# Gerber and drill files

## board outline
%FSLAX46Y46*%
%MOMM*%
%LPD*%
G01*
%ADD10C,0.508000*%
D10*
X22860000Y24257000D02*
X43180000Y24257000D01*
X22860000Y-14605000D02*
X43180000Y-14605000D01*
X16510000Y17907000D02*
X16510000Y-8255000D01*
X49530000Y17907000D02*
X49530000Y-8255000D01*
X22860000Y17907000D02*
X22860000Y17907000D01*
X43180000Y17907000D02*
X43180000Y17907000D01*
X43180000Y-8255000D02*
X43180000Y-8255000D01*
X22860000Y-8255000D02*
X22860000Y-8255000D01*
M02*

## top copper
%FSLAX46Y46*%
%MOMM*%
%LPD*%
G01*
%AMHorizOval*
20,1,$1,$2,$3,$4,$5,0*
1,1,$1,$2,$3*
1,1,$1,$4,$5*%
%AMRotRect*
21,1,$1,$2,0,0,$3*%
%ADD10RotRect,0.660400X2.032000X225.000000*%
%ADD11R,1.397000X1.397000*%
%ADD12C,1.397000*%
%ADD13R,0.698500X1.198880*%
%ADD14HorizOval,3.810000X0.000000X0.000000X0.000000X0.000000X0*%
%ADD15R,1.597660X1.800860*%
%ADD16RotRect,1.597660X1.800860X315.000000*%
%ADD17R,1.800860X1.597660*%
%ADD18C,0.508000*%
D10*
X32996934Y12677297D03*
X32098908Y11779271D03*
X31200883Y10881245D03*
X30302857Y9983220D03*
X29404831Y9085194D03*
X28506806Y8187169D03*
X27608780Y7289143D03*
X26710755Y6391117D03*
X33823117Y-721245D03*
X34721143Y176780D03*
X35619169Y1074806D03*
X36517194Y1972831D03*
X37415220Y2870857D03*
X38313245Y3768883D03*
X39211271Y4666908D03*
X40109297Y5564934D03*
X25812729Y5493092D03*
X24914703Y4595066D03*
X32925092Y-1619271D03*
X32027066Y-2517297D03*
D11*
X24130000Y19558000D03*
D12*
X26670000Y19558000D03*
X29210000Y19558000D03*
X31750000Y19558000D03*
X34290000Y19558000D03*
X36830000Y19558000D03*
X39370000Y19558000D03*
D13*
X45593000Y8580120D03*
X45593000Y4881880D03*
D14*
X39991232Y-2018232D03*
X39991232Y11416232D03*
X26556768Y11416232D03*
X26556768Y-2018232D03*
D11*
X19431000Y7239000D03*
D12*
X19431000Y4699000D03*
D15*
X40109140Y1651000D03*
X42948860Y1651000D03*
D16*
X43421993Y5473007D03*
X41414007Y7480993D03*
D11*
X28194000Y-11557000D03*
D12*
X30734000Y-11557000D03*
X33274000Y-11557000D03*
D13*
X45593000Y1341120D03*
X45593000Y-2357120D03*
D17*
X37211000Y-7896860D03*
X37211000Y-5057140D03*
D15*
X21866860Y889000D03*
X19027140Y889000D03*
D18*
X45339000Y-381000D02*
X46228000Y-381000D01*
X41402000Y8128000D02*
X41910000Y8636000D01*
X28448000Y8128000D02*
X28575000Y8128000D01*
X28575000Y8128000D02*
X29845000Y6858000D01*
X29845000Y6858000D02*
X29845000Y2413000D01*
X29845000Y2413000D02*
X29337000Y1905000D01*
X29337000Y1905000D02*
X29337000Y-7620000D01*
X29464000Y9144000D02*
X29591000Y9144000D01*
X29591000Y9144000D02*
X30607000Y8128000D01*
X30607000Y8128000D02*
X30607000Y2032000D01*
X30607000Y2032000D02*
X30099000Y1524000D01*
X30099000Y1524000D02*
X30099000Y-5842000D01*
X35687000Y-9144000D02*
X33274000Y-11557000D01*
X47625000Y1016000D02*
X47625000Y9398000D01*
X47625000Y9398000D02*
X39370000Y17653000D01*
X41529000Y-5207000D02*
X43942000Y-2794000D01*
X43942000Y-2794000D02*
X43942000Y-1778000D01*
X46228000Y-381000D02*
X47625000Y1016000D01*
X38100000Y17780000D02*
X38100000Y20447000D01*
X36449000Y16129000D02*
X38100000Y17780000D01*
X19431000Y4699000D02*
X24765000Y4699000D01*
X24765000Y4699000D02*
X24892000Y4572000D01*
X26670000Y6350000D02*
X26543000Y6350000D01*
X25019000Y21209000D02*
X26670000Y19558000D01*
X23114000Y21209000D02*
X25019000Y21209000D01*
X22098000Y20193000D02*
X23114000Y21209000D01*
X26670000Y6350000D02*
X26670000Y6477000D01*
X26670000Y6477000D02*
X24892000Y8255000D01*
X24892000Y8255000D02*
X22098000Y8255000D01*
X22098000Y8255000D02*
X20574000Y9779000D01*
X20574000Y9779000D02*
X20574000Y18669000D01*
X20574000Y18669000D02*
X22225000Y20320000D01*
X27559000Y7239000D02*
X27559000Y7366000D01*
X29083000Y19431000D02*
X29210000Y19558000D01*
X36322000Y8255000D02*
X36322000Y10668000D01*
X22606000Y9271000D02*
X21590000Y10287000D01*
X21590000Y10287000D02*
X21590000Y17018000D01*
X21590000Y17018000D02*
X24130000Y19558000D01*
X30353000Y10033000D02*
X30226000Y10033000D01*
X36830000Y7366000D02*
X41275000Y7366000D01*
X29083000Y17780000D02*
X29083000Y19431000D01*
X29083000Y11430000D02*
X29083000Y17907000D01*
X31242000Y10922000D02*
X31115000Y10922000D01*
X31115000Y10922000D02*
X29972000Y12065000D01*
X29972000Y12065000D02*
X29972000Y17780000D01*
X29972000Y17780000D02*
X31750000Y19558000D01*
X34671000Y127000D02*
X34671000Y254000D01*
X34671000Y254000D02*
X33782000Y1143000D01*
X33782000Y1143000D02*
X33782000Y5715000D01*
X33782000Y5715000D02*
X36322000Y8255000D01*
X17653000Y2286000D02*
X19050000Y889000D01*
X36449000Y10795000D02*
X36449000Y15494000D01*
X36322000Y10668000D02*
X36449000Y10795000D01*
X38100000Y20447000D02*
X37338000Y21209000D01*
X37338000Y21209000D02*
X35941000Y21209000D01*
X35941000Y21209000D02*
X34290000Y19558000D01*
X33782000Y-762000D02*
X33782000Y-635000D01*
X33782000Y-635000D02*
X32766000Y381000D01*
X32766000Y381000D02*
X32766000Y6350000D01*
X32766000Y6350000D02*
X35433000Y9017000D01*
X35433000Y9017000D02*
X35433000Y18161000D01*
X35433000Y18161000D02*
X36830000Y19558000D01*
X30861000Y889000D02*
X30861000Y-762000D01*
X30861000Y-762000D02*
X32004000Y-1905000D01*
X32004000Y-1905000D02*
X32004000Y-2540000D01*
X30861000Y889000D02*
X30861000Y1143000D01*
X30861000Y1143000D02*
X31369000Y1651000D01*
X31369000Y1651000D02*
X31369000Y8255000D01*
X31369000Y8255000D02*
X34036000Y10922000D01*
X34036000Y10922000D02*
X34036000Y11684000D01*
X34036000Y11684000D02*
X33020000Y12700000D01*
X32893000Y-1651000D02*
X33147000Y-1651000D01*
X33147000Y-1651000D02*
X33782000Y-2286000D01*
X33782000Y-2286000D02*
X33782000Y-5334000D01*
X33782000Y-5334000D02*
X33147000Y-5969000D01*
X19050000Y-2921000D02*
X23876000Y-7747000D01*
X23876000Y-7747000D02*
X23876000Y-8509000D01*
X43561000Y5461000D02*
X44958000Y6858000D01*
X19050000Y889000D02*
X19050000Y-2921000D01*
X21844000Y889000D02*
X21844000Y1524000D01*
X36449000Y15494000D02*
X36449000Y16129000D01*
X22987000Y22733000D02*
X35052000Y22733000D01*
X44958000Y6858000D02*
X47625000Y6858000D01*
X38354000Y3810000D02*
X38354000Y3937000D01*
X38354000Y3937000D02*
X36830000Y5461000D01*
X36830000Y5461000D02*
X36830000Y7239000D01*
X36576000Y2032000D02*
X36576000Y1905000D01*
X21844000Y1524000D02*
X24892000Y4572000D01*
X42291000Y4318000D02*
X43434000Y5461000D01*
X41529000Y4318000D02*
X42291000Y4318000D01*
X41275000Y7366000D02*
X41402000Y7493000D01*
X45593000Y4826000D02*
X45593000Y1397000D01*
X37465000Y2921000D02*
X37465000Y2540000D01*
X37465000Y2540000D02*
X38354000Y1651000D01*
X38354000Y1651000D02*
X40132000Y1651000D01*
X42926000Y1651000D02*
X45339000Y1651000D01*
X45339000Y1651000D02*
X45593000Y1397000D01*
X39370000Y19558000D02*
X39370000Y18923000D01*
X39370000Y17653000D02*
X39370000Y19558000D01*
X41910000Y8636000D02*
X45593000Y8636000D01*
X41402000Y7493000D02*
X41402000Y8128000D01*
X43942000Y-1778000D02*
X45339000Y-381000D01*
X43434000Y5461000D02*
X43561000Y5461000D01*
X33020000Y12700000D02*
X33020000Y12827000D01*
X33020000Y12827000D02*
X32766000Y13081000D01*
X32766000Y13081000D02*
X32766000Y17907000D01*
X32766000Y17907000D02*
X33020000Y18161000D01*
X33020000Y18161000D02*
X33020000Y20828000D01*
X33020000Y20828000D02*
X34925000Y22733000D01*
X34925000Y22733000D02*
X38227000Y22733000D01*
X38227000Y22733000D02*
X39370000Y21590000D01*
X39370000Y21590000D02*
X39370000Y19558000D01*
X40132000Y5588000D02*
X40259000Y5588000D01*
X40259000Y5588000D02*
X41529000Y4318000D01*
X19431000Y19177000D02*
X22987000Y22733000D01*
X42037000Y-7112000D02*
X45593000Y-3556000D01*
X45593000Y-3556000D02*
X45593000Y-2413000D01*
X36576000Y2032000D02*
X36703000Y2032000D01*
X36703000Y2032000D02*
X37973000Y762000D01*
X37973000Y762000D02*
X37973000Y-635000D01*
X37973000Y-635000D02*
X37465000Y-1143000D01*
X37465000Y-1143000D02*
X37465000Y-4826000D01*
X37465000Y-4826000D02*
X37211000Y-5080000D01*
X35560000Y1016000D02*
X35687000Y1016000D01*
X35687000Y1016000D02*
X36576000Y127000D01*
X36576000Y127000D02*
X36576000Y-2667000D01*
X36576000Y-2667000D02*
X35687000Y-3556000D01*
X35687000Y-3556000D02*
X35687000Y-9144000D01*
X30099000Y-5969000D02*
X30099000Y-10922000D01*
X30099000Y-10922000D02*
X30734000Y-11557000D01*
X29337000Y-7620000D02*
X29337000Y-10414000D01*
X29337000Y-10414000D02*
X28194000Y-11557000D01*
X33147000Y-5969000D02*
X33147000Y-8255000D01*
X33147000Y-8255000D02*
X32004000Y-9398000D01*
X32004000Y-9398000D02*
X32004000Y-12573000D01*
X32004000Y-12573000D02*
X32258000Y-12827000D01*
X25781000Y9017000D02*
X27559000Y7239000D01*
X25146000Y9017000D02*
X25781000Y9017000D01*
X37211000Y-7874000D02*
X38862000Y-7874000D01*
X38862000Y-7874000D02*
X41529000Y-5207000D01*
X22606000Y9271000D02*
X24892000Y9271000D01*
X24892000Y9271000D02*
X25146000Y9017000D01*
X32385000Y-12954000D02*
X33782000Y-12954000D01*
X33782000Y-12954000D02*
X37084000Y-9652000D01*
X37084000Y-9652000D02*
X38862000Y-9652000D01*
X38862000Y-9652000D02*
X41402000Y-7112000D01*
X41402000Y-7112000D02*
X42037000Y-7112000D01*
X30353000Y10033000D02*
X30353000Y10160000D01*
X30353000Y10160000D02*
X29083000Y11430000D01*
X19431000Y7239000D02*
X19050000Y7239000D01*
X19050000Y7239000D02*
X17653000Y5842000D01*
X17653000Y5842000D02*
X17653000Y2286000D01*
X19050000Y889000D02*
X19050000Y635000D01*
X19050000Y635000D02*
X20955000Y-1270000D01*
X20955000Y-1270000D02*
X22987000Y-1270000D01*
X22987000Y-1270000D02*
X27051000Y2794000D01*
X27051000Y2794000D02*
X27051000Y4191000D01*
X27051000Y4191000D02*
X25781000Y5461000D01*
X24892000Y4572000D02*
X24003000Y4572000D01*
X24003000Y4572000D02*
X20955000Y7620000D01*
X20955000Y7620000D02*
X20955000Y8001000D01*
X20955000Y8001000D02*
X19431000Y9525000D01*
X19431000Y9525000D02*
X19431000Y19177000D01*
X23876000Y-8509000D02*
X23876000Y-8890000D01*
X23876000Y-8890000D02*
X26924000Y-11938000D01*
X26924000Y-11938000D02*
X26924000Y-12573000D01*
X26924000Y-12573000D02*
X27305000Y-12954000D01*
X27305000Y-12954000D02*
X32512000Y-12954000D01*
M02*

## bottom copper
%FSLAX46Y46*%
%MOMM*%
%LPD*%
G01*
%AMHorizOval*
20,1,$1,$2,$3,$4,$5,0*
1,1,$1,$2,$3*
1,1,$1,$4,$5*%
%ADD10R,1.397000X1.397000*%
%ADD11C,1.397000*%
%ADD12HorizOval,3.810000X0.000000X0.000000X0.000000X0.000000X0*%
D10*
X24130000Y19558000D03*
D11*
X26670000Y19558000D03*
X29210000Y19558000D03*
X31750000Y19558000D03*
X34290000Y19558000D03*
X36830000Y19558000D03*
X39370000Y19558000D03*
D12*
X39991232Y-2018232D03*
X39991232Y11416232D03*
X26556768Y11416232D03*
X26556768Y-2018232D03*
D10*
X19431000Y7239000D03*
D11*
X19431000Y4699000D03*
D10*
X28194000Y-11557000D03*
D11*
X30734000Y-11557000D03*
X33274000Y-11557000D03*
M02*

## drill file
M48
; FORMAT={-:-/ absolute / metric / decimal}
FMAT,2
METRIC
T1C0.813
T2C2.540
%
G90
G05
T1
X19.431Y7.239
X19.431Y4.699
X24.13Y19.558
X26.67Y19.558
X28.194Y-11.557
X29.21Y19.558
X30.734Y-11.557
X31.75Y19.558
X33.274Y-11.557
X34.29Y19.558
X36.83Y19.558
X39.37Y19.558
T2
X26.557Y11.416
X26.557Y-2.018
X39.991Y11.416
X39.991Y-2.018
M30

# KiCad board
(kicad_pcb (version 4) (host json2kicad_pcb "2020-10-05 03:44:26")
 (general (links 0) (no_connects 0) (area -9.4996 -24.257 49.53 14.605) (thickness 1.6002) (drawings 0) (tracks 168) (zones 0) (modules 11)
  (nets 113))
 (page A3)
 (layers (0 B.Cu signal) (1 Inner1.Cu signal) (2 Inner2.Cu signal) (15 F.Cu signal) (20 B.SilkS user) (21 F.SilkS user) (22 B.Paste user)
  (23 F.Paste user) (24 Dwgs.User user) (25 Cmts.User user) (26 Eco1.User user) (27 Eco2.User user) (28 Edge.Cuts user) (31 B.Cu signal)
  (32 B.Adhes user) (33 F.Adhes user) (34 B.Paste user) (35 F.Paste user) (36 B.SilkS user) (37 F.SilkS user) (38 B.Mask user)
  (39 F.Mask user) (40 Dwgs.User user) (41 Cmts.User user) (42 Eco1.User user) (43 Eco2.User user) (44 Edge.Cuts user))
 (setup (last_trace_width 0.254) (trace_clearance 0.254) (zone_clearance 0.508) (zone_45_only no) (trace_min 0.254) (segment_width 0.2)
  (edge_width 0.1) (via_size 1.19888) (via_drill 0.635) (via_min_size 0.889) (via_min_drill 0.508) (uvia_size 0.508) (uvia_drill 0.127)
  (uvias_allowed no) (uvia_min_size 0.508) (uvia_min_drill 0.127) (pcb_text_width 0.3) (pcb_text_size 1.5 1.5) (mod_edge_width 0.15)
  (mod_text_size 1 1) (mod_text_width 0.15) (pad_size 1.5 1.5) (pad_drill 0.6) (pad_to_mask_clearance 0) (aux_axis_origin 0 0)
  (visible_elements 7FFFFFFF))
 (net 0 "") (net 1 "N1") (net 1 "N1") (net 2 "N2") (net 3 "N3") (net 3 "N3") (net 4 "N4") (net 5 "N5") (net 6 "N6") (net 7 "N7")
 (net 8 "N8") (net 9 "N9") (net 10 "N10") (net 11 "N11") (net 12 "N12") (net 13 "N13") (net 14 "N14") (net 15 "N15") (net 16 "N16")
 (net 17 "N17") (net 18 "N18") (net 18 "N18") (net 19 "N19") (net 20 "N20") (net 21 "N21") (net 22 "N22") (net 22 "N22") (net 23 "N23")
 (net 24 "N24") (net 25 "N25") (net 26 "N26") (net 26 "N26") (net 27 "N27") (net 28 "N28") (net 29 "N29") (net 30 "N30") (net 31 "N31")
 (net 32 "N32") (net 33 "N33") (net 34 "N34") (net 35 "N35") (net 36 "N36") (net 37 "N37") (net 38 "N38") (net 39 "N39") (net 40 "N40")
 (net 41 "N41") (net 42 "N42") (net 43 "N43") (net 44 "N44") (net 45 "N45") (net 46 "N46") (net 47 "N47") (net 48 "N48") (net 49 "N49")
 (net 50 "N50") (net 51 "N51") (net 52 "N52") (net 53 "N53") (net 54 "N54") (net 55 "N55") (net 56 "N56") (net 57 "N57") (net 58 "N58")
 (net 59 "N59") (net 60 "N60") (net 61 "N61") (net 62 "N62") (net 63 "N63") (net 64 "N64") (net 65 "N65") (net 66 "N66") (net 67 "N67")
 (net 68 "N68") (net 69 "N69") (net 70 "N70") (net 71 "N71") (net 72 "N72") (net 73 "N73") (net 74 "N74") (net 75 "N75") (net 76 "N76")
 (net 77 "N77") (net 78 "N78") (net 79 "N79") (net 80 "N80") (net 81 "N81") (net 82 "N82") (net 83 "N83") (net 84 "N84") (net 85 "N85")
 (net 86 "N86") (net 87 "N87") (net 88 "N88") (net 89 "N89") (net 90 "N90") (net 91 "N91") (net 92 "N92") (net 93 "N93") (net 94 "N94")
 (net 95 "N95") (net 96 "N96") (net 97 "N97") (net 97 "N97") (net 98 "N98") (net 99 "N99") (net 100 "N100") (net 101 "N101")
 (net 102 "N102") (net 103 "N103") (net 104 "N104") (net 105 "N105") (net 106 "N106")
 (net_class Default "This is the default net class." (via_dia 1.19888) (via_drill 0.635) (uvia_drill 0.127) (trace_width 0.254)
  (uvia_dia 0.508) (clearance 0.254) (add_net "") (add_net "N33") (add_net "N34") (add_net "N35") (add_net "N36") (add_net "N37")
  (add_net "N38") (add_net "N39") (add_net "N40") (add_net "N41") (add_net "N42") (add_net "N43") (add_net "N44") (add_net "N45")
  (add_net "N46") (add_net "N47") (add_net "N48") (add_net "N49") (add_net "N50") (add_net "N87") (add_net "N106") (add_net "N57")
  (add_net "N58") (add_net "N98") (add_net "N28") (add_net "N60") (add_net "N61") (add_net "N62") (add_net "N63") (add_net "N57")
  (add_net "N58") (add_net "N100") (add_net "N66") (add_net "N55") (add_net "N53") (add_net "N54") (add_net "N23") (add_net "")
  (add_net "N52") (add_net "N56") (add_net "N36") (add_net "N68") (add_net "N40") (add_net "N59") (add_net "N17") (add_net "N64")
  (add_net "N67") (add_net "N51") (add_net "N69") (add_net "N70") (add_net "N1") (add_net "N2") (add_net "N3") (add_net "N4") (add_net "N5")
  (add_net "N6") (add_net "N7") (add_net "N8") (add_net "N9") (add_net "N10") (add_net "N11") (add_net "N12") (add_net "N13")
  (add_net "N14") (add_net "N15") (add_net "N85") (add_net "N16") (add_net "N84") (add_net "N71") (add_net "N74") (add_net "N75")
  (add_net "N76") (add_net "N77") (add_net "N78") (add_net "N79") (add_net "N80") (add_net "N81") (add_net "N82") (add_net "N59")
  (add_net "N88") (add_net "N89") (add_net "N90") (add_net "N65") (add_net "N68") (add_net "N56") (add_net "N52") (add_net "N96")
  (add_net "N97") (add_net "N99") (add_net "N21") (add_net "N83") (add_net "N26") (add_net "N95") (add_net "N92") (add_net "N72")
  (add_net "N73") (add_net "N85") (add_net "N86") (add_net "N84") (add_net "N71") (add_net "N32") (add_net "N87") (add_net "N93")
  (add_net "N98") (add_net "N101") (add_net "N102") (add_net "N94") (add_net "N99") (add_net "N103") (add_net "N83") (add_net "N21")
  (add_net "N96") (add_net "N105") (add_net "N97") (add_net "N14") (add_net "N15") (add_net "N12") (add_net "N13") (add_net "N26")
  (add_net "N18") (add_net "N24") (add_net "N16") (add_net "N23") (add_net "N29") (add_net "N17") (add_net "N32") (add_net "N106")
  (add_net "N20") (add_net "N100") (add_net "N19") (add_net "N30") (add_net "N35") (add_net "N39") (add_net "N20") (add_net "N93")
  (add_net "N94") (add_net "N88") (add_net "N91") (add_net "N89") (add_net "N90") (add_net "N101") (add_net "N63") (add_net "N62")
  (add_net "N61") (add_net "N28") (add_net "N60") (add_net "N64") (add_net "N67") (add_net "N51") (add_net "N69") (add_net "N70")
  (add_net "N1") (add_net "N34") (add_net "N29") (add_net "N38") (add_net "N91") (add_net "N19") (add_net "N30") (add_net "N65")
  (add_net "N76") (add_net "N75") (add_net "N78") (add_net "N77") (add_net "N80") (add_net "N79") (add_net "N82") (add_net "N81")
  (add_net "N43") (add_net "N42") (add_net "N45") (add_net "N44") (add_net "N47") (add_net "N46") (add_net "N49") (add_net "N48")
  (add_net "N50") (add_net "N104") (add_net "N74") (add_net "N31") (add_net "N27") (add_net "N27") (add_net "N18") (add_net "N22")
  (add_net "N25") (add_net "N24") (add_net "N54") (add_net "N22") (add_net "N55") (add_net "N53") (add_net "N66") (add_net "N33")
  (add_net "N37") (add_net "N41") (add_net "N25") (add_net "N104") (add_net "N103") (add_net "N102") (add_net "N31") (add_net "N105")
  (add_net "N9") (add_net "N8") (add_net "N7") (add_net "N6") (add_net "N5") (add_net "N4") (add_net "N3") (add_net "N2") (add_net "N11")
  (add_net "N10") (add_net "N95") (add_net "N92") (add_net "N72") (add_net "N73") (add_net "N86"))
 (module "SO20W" (layer "F.Cu") (at 32.512 -5.08 -135.00)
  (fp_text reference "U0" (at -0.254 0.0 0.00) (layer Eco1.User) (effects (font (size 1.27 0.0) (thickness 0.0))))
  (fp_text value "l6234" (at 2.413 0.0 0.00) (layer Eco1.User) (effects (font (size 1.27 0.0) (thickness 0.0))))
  (pad 1 smd rect (at -5.715 5.0292 -135.00) (size 0.6604 2.032) (drill 0.0) (layers "F.Cu" "F.Paste") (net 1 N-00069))
  (pad 2 smd rect (at -4.445 5.0292 -135.00) (size 0.6604 2.032) (drill 0.0) (layers "F.Cu" "F.Paste") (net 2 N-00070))
  (pad 3 smd rect (at -3.175 5.0292 -135.00) (size 0.6604 2.032) (drill 0.0) (layers "F.Cu" "F.Paste") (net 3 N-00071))
  (pad 4 smd rect (at -1.905 5.0292 -135.00) (size 0.6604 2.032) (drill 0.0) (layers "F.Cu" "F.Paste") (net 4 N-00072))
  (pad 5 smd rect (at -0.635 5.0292 -135.00) (size 0.6604 2.032) (drill 0.0) (layers "F.Cu" "F.Paste") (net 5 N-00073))
  (pad 6 smd rect (at 0.635 5.0292 -135.00) (size 0.6604 2.032) (drill 0.0) (layers "F.Cu" "F.Paste") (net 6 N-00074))
  (pad 7 smd rect (at 1.905 5.0292 -135.00) (size 0.6604 2.032) (drill 0.0) (layers "F.Cu" "F.Paste") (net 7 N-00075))
  (pad 8 smd rect (at 3.175 5.0292 -135.00) (size 0.6604 2.032) (drill 0.0) (layers "F.Cu" "F.Paste") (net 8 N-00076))
  (pad 13 smd rect (at 3.175 -5.0292 -135.00) (size 0.6604 2.032) (drill 0.0) (layers "F.Cu" "F.Paste") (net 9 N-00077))
  (pad 14 smd rect (at 1.905 -5.0292 -135.00) (size 0.6604 2.032) (drill 0.0) (layers "F.Cu" "F.Paste") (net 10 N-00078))
  (pad 15 smd rect (at 0.635 -5.0292 -135.00) (size 0.6604 2.032) (drill 0.0) (layers "F.Cu" "F.Paste") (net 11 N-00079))
  (pad 16 smd rect (at -0.635 -5.0292 -135.00) (size 0.6604 2.032) (drill 0.0) (layers "F.Cu" "F.Paste") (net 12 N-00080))
  (pad 17 smd rect (at -1.905 -5.0292 -135.00) (size 0.6604 2.032) (drill 0.0) (layers "F.Cu" "F.Paste") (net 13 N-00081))
  (pad 18 smd rect (at -3.175 -5.0292 -135.00) (size 0.6604 2.032) (drill 0.0) (layers "F.Cu" "F.Paste") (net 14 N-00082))
  (pad 19 smd rect (at -4.445 -5.0292 -135.00) (size 0.6604 2.032) (drill 0.0) (layers "F.Cu" "F.Paste") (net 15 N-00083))
  (pad 20 smd rect (at -5.715 -5.0292 -135.00) (size 0.6604 2.032) (drill 0.0) (layers "F.Cu" "F.Paste") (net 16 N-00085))
  (pad 9 smd rect (at 4.445 5.0292 -135.00) (size 0.6604 2.032) (drill 0.0) (layers "F.Cu" "F.Paste") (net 16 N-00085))
  (pad 10 smd rect (at 5.715 5.0292 -135.00) (size 0.6604 2.032) (drill 0.0) (layers "F.Cu" "F.Paste") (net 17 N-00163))
  (pad 12 smd rect (at 4.445 -5.0292 -135.00) (size 0.6604 2.032) (drill 0.0) (layers "F.Cu" "F.Paste") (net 6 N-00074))
  (pad 11 smd rect (at 5.715 -5.0292 -135.00) (size 0.6604 2.032) (drill 0.0) (layers "F.Cu" "F.Paste") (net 1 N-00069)))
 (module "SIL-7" (layer "F.Cu") (at 31.75 -19.558 0.00)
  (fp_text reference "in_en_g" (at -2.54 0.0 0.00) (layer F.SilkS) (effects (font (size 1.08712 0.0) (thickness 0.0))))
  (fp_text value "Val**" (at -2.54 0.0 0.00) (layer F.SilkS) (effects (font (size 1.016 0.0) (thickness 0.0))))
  (pad 1 thru_hole rect (at -7.62 0.0 0.00) (size 1.397 1.397) (drill 0.8128)
   (layers "B.Cu" "Inner1.Cu" "Inner2.Cu" "F.Cu" "F.SilkS" "B.Paste" "F.Paste") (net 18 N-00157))
  (pad 2 thru_hole circle (at -5.08 0.0 0.00) (size 1.397 1.397) (drill 0.8128)
   (layers "B.Cu" "Inner1.Cu" "Inner2.Cu" "F.Cu" "B.SilkS" "F.SilkS" "B.Paste" "F.Paste") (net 8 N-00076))
  (pad 3 thru_hole circle (at -2.54 0.0 0.00) (size 1.397 1.397) (drill 0.8128)
   (layers "B.Cu" "Inner1.Cu" "Inner2.Cu" "F.Cu" "B.SilkS" "F.SilkS" "B.Paste" "F.Paste") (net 7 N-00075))
  (pad 4 thru_hole circle (at 0.0 0.0 0.00) (size 1.397 1.397) (drill 0.8128)
   (layers "B.Cu" "Inner1.Cu" "Inner2.Cu" "F.Cu" "B.SilkS" "F.SilkS" "B.Paste" "F.Paste") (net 3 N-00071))
  (pad 5 thru_hole circle (at 2.54 0.0 0.00) (size 1.397 1.397) (drill 0.8128)
   (layers "B.Cu" "Inner1.Cu" "Inner2.Cu" "F.Cu" "B.SilkS" "F.SilkS" "B.Paste" "F.Paste") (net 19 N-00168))
  (pad 6 thru_hole circle (at 5.08 0.0 0.00) (size 1.397 1.397) (drill 0.8128)
   (layers "B.Cu" "Inner1.Cu" "Inner2.Cu" "F.Cu" "B.SilkS" "F.SilkS" "B.Paste" "F.Paste") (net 9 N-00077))
  (pad 7 thru_hole circle (at 7.62 0.0 0.00) (size 1.397 1.397) (drill 0.8128)
   (layers "B.Cu" "Inner1.Cu" "Inner2.Cu" "F.Cu" "B.SilkS" "F.SilkS" "B.Paste" "F.Paste") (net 1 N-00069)))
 (segment (start 45.339 0.381) (end 46.228 0.381) (width 0.508) (layer F.Cu) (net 1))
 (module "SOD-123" (layer "F.Cu") (at 45.593 -6.731 -90.00)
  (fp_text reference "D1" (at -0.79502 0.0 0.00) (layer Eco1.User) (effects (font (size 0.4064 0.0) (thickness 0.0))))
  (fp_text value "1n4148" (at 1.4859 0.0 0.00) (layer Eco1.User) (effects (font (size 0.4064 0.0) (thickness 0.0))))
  (pad C smd rect (at -1.84912 0.0 -90.00) (size 1.19888 0.6985) (drill 0.0) (layers "F.Cu" "F.Paste") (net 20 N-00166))
  (pad A smd rect (at 1.84912 0.0 -90.00) (size 1.19888 0.6985) (drill 0.0) (layers "F.Cu" "F.Paste") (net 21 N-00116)))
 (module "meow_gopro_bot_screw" (layer "F.Cu") (at 33.274 -4.699 45.00)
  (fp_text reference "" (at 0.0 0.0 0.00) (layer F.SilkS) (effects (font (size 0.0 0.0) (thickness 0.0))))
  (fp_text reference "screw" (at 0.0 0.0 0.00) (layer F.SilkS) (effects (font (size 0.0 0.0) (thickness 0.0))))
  (pad S0 thru_hole oval (at 0.0 9.4996 45.00) (size 3.81 3.81) (drill 2.54)
   (layers "B.Cu" "Inner1.Cu" "Inner2.Cu" "F.Cu" "B.Paste" "F.Paste") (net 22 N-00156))
  (pad S1 thru_hole oval (at 9.4996 0.0 45.00) (size 3.81 3.81) (drill 2.54)
   (layers "B.Cu" "Inner1.Cu" "Inner2.Cu" "F.Cu" "B.Paste" "F.Paste") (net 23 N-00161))
  (pad S2 thru_hole oval (at 0.0 -9.4996 45.00) (size 3.81 3.81) (drill 2.54)
   (layers "B.Cu" "Inner1.Cu" "Inner2.Cu" "F.Cu" "B.Paste" "F.Paste") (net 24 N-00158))
  (pad S3 thru_hole oval (at -9.4996 0.0 45.00) (size 3.81 3.81) (drill 2.54)
   (layers "B.Cu" "Inner1.Cu" "Inner2.Cu" "F.Cu" "B.Paste" "F.Paste") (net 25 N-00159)))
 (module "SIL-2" (layer "F.Cu") (at 19.431 -5.969 -90.00)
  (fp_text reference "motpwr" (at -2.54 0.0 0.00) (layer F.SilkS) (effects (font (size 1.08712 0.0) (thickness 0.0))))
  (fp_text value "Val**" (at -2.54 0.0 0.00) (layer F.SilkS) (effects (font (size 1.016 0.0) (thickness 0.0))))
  (pad 1 thru_hole rect (at -1.27 0.0 -90.00) (size 1.397 1.397) (drill 0.8128)
   (layers "B.Cu" "Inner1.Cu" "Inner2.Cu" "F.Cu" "F.SilkS" "B.Paste" "F.Paste") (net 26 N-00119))
  (pad 2 thru_hole circle (at 1.27 0.0 -90.00) (size 1.397 1.397) (drill 0.8128)
   (layers "B.Cu" "Inner1.Cu" "Inner2.Cu" "F.Cu" "F.SilkS" "B.Paste" "F.Paste") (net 17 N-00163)))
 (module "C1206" (layer "F.Cu") (at 41.529 -1.651 180.00)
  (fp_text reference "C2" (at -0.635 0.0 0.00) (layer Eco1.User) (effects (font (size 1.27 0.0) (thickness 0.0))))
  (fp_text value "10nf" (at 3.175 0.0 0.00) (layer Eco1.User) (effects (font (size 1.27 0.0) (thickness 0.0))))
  (pad 2 smd rect (at 1.41986 0.0 -180.00) (size 1.59766 1.80086) (drill 0.0) (layers "F.Cu" "F.Paste") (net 13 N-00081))
  (pad 1 smd rect (at -1.41986 0.0 -180.00) (size 1.59766 1.80086) (drill 0.0) (layers "F.Cu" "F.Paste") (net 21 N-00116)))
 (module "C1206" (layer "F.Cu") (at 42.418 -6.477 -45.00)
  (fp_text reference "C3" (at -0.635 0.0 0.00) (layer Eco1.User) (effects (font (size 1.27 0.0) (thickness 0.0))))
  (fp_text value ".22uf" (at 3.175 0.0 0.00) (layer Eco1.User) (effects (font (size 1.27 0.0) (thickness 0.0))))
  (pad 2 smd rect (at 1.41986 0.0 -45.00) (size 1.59766 1.80086) (drill 0.0) (layers "F.Cu" "F.Paste") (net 16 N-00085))
  (pad 1 smd rect (at -1.41986 0.0 -45.00) (size 1.59766 1.80086) (drill 0.0) (layers "F.Cu" "F.Paste") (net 12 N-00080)))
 (segment (start 41.402 -8.128) (end 41.91 -8.636) (width 0.508) (layer F.Cu) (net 14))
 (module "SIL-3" (layer "F.Cu") (at 30.734 11.557 0.00)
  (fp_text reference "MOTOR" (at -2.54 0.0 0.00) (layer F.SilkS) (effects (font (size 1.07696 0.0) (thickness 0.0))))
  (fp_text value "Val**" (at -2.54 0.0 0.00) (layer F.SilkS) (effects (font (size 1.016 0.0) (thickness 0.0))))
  (pad 1 thru_hole rect (at -2.54 0.0 0.00) (size 1.397 1.397) (drill 0.8128)
   (layers "B.Cu" "Inner1.Cu" "Inner2.Cu" "F.Cu" "F.SilkS" "B.Paste" "F.Paste") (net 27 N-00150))
  (pad 2 thru_hole circle (at 0.0 0.0 0.00) (size 1.397 1.397) (drill 0.8128)
   (layers "B.Cu" "Inner1.Cu" "Inner2.Cu" "F.Cu" "F.SilkS" "B.Paste" "F.Paste") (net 5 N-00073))
  (pad 3 thru_hole circle (at 2.54 0.0 0.00) (size 1.397 1.397) (drill 0.8128)
   (layers "B.Cu" "Inner1.Cu" "Inner2.Cu" "F.Cu" "F.SilkS" "B.Paste" "F.Paste") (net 11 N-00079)))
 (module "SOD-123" (layer "F.Cu") (at 45.593 0.508 -90.00)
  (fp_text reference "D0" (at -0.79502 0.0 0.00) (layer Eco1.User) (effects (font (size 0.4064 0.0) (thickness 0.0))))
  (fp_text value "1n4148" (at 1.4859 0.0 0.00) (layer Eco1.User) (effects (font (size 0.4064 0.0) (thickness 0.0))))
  (pad C smd rect (at -1.84912 0.0 -90.00) (size 1.19888 0.6985) (drill 0.0) (layers "F.Cu" "F.Paste") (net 1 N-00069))
  (pad A smd rect (at 1.84912 0.0 -90.00) (size 1.19888 0.6985) (drill 0.0) (layers "F.Cu" "F.Paste") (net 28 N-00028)))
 (segment (start 28.448 -8.128) (end 28.575 -8.128) (width 0.508) (layer F.Cu) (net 6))
 (segment (start 28.575 -8.128) (end 29.845 -6.858) (width 0.508) (layer F.Cu) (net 6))
 (segment (start 29.845 -6.858) (end 29.845 -2.413) (width 0.508) (layer F.Cu) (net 6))
 (segment (start 29.845 -2.413) (end 29.337 -1.905) (width 0.508) (layer F.Cu) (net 6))
 (segment (start 29.337 -1.905) (end 29.337 7.62) (width 0.508) (layer F.Cu) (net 6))
 (segment (start 29.464 -9.144) (end 29.591 -9.144) (width 0.508) (layer F.Cu) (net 5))
 (segment (start 29.591 -9.144) (end 30.607 -8.128) (width 0.508) (layer F.Cu) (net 5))
 (segment (start 30.607 -8.128) (end 30.607 -2.032) (width 0.508) (layer F.Cu) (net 5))
 (segment (start 30.607 -2.032) (end 30.099 -1.524) (width 0.508) (layer F.Cu) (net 5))
 (segment (start 30.099 -1.524) (end 30.099 5.842) (width 0.508) (layer F.Cu) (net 5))
 (segment (start 35.687 9.144) (end 33.274 11.557) (width 0.508) (layer F.Cu) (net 11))
 (segment (start 47.625 -1.016) (end 47.625 -9.398) (width 0.508) (layer F.Cu) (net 1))
 (segment (start 47.625 -9.398) (end 39.37 -17.653) (width 0.508) (layer F.Cu) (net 1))
 (segment (start 41.529 5.207) (end 43.942 2.794) (width 0.508) (layer F.Cu) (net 1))
 (segment (start 43.942 2.794) (end 43.942 1.778) (width 0.508) (layer F.Cu) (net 1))
 (segment (start 46.228 0.381) (end 47.625 -1.016) (width 0.508) (layer F.Cu) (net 1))
 (segment (start 38.1 -17.78) (end 38.1 -20.447) (width 0.508) (layer F.Cu) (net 10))
 (segment (start 36.449 -16.129) (end 38.1 -17.78) (width 0.508) (layer F.Cu) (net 10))
 (segment (start 19.431 -4.699) (end 24.765 -4.699) (width 0.508) (layer F.Cu) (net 17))
 (segment (start 24.765 -4.699) (end 24.892 -4.572) (width 0.508) (layer F.Cu) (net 17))
 (segment (start 26.67 -6.35) (end 26.543 -6.35) (width 0.508) (layer F.Cu) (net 8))
 (segment (start 25.019 -21.209) (end 26.67 -19.558) (width 0.508) (layer F.Cu) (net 8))
 (segment (start 23.114 -21.209) (end 25.019 -21.209) (width 0.508) (layer F.Cu) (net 8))
 (segment (start 22.098 -20.193) (end 23.114 -21.209) (width 0.508) (layer F.Cu) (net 8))
 (segment (start 26.67 -6.35) (end 26.67 -6.477) (width 0.508) (layer F.Cu) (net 8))
 (segment (start 26.67 -6.477) (end 24.892 -8.255) (width 0.508) (layer F.Cu) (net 8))
 (segment (start 24.892 -8.255) (end 22.098 -8.255) (width 0.508) (layer F.Cu) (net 8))
 (segment (start 22.098 -8.255) (end 20.574 -9.779) (width 0.508) (layer F.Cu) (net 8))
 (segment (start 20.574 -9.779) (end 20.574 -18.669) (width 0.508) (layer F.Cu) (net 8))
 (segment (start 20.574 -18.669) (end 22.225 -20.32) (width 0.508) (layer F.Cu) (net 8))
 (segment (start 27.559 -7.239) (end 27.559 -7.366) (width 0.508) (layer F.Cu) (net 7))
 (segment (start 29.083 -19.431) (end 29.21 -19.558) (width 0.508) (layer F.Cu) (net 4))
 (segment (start 36.322 -8.255) (end 36.322 -10.668) (width 0.508) (layer F.Cu) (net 10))
 (segment (start 22.606 -9.271) (end 21.59 -10.287) (width 0.508) (layer F.Cu) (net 18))
 (segment (start 21.59 -10.287) (end 21.59 -17.018) (width 0.508) (layer F.Cu) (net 18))
 (segment (start 21.59 -17.018) (end 24.13 -19.558) (width 0.508) (layer F.Cu) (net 18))
 (segment (start 30.353 -10.033) (end 30.226 -10.033) (width 0.508) (layer F.Cu) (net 4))
 (segment (start 36.83 -7.366) (end 41.275 -7.366) (width 0.508) (layer F.Cu) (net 14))
 (segment (start 29.083 -17.78) (end 29.083 -19.431) (width 0.508) (layer F.Cu) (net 4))
 (segment (start 29.083 -11.43) (end 29.083 -17.907) (width 0.508) (layer F.Cu) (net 4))
 (segment (start 31.242 -10.922) (end 31.115 -10.922) (width 0.508) (layer F.Cu) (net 3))
 (segment (start 31.115 -10.922) (end 29.972 -12.065) (width 0.508) (layer F.Cu) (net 3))
 (segment (start 29.972 -12.065) (end 29.972 -17.78) (width 0.508) (layer F.Cu) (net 3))
 (segment (start 29.972 -17.78) (end 31.75 -19.558) (width 0.508) (layer F.Cu) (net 3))
 (segment (start 34.671 -0.127) (end 34.671 -0.254) (width 0.508) (layer F.Cu) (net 10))
 (segment (start 34.671 -0.254) (end 33.782 -1.143) (width 0.508) (layer F.Cu) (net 10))
 (segment (start 33.782 -1.143) (end 33.782 -5.715) (width 0.508) (layer F.Cu) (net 10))
 (segment (start 33.782 -5.715) (end 36.322 -8.255) (width 0.508) (layer F.Cu) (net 10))
 (segment (start 17.653 -2.286) (end 19.05 -0.889) (width 0.508) (layer F.Cu) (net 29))
 (segment (start 36.449 -10.795) (end 36.449 -15.494) (width 0.508) (layer F.Cu) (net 10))
 (segment (start 36.322 -10.668) (end 36.449 -10.795) (width 0.508) (layer F.Cu) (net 10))
 (segment (start 38.1 -20.447) (end 37.338 -21.209) (width 0.508) (layer F.Cu) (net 19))
 (segment (start 37.338 -21.209) (end 35.941 -21.209) (width 0.508) (layer F.Cu) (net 19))
 (segment (start 35.941 -21.209) (end 34.29 -19.558) (width 0.508) (layer F.Cu) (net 19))
 (segment (start 33.782 0.762) (end 33.782 0.635) (width 0.508) (layer F.Cu) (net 9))
 (segment (start 33.782 0.635) (end 32.766 -0.381) (width 0.508) (layer F.Cu) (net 9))
 (segment (start 32.766 -0.381) (end 32.766 -6.35) (width 0.508) (layer F.Cu) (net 9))
 (segment (start 32.766 -6.35) (end 35.433 -9.017) (width 0.508) (layer F.Cu) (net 9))
 (segment (start 35.433 -9.017) (end 35.433 -18.161) (width 0.508) (layer F.Cu) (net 9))
 (segment (start 35.433 -18.161) (end 36.83 -19.558) (width 0.508) (layer F.Cu) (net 9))
 (segment (start 30.861 -0.889) (end 30.861 0.762) (width 0.508) (layer F.Cu) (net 1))
 (segment (start 30.861 0.762) (end 32.004 1.905) (width 0.508) (layer F.Cu) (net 1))
 (segment (start 32.004 1.905) (end 32.004 2.54) (width 0.508) (layer F.Cu) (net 1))
 (segment (start 30.861 -0.889) (end 30.861 -1.143) (width 0.508) (layer F.Cu) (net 1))
 (segment (start 30.861 -1.143) (end 31.369 -1.651) (width 0.508) (layer F.Cu) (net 1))
 (segment (start 31.369 -1.651) (end 31.369 -8.255) (width 0.508) (layer F.Cu) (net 1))
 (segment (start 31.369 -8.255) (end 34.036 -10.922) (width 0.508) (layer F.Cu) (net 1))
 (segment (start 34.036 -10.922) (end 34.036 -11.684) (width 0.508) (layer F.Cu) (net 1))
 (segment (start 34.036 -11.684) (end 33.02 -12.7) (width 0.508) (layer F.Cu) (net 1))
 (segment (start 32.893 1.651) (end 33.147 1.651) (width 0.508) (layer F.Cu) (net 6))
 (segment (start 33.147 1.651) (end 33.782 2.286) (width 0.508) (layer F.Cu) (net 6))
 (segment (start 33.782 2.286) (end 33.782 5.334) (width 0.508) (layer F.Cu) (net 6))
 (segment (start 33.782 5.334) (end 33.147 5.969) (width 0.508) (layer F.Cu) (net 6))
 (segment (start 19.05 2.921) (end 23.876 7.747) (width 0.508) (layer F.Cu) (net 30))
 (segment (start 23.876 7.747) (end 23.876 8.509) (width 0.508) (layer F.Cu) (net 30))
 (segment (start 43.561 -5.461) (end 44.958 -6.858) (width 0.508) (layer F.Cu) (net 1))
 (segment (start 19.05 -0.889) (end 19.05 2.921) (width 0.508) (layer F.Cu) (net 30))
 (segment (start 21.844 -0.889) (end 21.844 -1.524) (width 0.508) (layer F.Cu) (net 17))
 (segment (start 36.449 -15.494) (end 36.449 -16.129) (width 0.508) (layer F.Cu) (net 10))
 (segment (start 22.987 -22.733) (end 35.052 -22.733) (width 0.508) (layer F.Cu) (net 1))
 (segment (start 44.958 -6.858) (end 47.625 -6.858) (width 0.508) (layer F.Cu) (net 1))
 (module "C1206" (layer "F.Cu") (at 37.211 6.477 -90.00)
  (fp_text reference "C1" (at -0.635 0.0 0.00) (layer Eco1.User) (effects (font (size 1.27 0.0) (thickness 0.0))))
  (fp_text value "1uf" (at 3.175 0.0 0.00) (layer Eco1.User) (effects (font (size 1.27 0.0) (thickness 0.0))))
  (pad 2 smd rect (at 1.41986 0.0 -90.00) (size 1.59766 1.80086) (drill 0.0) (layers "F.Cu" "F.Paste") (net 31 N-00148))
  (pad 1 smd rect (at -1.41986 0.0 -90.00) (size 1.59766 1.80086) (drill 0.0) (layers "F.Cu" "F.Paste") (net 29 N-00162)))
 (segment (start 38.354 -3.81) (end 38.354 -3.937) (width 0.508) (layer F.Cu) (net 14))
 (segment (start 38.354 -3.937) (end 36.83 -5.461) (width 0.508) (layer F.Cu) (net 14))
 (segment (start 36.83 -5.461) (end 36.83 -7.239) (width 0.508) (layer F.Cu) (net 14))
 (segment (start 36.576 -2.032) (end 36.576 -1.905) (width 0.508) (layer F.Cu) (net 12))
 (segment (start 21.844 -1.524) (end 24.892 -4.572) (width 0.508) (layer F.Cu) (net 17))
 (segment (start 42.291 -4.318) (end 43.434 -5.461) (width 0.508) (layer F.Cu) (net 16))
 (segment (start 41.529 -4.318) (end 42.291 -4.318) (width 0.508) (layer F.Cu) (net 16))
 (segment (start 41.275 -7.366) (end 41.402 -7.493) (width 0.508) (layer F.Cu) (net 14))
 (segment (start 45.593 -4.826) (end 45.593 -1.397) (width 0.508) (layer F.Cu) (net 21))
 (segment (start 37.465 -2.921) (end 37.465 -2.54) (width 0.508) (layer F.Cu) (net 13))
 (segment (start 37.465 -2.54) (end 38.354 -1.651) (width 0.508) (layer F.Cu) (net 13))
 (segment (start 38.354 -1.651) (end 40.132 -1.651) (width 0.508) (layer F.Cu) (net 13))
 (segment (start 42.926 -1.651) (end 45.339 -1.651) (width 0.508) (layer F.Cu) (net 21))
 (segment (start 45.339 -1.651) (end 45.593 -1.397) (width 0.508) (layer F.Cu) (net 21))
 (segment (start 39.37 -19.558) (end 39.37 -18.923) (width 0.508) (layer F.Cu) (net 1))
 (segment (start 39.37 -17.653) (end 39.37 -19.558) (width 0.508) (layer F.Cu) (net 1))
 (segment (start 41.91 -8.636) (end 45.593 -8.636) (width 0.508) (layer F.Cu) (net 14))
 (segment (start 41.402 -7.493) (end 41.402 -8.128) (width 0.508) (layer F.Cu) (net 14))
 (segment (start 43.942 1.778) (end 45.339 0.381) (width 0.508) (layer F.Cu) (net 1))
 (segment (start 43.434 -5.461) (end 43.561 -5.461) (width 0.508) (layer F.Cu) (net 1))
 (segment (start 33.02 -12.7) (end 33.02 -12.827) (width 0.508) (layer F.Cu) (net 1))
 (segment (start 33.02 -12.827) (end 32.766 -13.081) (width 0.508) (layer F.Cu) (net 1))
 (segment (start 32.766 -13.081) (end 32.766 -17.907) (width 0.508) (layer F.Cu) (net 1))
 (segment (start 32.766 -17.907) (end 33.02 -18.161) (width 0.508) (layer F.Cu) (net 1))
 (segment (start 33.02 -18.161) (end 33.02 -20.828) (width 0.508) (layer F.Cu) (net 1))
 (segment (start 33.02 -20.828) (end 34.925 -22.733) (width 0.508) (layer F.Cu) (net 1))
 (segment (start 34.925 -22.733) (end 38.227 -22.733) (width 0.508) (layer F.Cu) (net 1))
 (segment (start 38.227 -22.733) (end 39.37 -21.59) (width 0.508) (layer F.Cu) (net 1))
 (segment (start 39.37 -21.59) (end 39.37 -19.558) (width 0.508) (layer F.Cu) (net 1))
 (segment (start 40.132 -5.588) (end 40.259 -5.588) (width 0.508) (layer F.Cu) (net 16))
 (segment (start 40.259 -5.588) (end 41.529 -4.318) (width 0.508) (layer F.Cu) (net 16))
 (segment (start 19.431 -19.177) (end 22.987 -22.733) (width 0.508) (layer F.Cu) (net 1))
 (segment (start 42.037 7.112) (end 45.593 3.556) (width 0.508) (layer F.Cu) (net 1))
 (segment (start 45.593 3.556) (end 45.593 2.413) (width 0.508) (layer F.Cu) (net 1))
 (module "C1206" (layer "F.Cu") (at 20.447 -0.889 0.00)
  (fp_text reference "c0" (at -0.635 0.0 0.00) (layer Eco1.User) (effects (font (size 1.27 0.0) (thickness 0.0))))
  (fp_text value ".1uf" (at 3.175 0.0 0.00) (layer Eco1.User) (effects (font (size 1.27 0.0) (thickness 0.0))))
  (pad 2 smd rect (at 1.41986 0.0 0.00) (size 1.59766 1.80086) (drill 0.0) (layers "F.Cu" "F.Paste") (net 17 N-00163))
  (pad 1 smd rect (at -1.41986 0.0 0.00) (size 1.59766 1.80086) (drill 0.0) (layers "F.Cu" "F.Paste") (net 30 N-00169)))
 (segment (start 36.576 -2.032) (end 36.703 -2.032) (width 0.508) (layer F.Cu) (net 12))
 (segment (start 36.703 -2.032) (end 37.973 -0.762) (width 0.508) (layer F.Cu) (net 12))
 (segment (start 37.973 -0.762) (end 37.973 0.635) (width 0.508) (layer F.Cu) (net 12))
 (segment (start 37.973 0.635) (end 37.465 1.143) (width 0.508) (layer F.Cu) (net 12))
 (segment (start 37.465 1.143) (end 37.465 4.826) (width 0.508) (layer F.Cu) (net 12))
 (segment (start 37.465 4.826) (end 37.211 5.08) (width 0.508) (layer F.Cu) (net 12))
 (segment (start 35.56 -1.016) (end 35.687 -1.016) (width 0.508) (layer F.Cu) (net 11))
 (segment (start 35.687 -1.016) (end 36.576 -0.127) (width 0.508) (layer F.Cu) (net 11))
 (segment (start 36.576 -0.127) (end 36.576 2.667) (width 0.508) (layer F.Cu) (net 11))
 (segment (start 36.576 2.667) (end 35.687 3.556) (width 0.508) (layer F.Cu) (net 11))
 (segment (start 35.687 3.556) (end 35.687 9.144) (width 0.508) (layer F.Cu) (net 11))
 (segment (start 30.099 5.969) (end 30.099 10.922) (width 0.508) (layer F.Cu) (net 5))
 (segment (start 30.099 10.922) (end 30.734 11.557) (width 0.508) (layer F.Cu) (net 5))
 (segment (start 29.337 7.62) (end 29.337 10.414) (width 0.508) (layer F.Cu) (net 6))
 (segment (start 29.337 10.414) (end 28.194 11.557) (width 0.508) (layer F.Cu) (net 6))
 (segment (start 33.147 5.969) (end 33.147 8.255) (width 0.508) (layer F.Cu) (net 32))
 (segment (start 33.147 8.255) (end 32.004 9.398) (width 0.508) (layer F.Cu) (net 32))
 (segment (start 32.004 9.398) (end 32.004 12.573) (width 0.508) (layer F.Cu) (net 32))
 (segment (start 32.004 12.573) (end 32.258 12.827) (width 0.508) (layer F.Cu) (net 32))
 (segment (start 25.781 -9.017) (end 27.559 -7.239) (width 0.508) (layer F.Cu) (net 7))
 (segment (start 25.146 -9.017) (end 25.781 -9.017) (width 0.508) (layer F.Cu) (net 7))
 (segment (start 37.211 7.874) (end 38.862 7.874) (width 0.508) (layer F.Cu) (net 1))
 (segment (start 38.862 7.874) (end 41.529 5.207) (width 0.508) (layer F.Cu) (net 1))
 (segment (start 22.606 -9.271) (end 24.892 -9.271) (width 0.508) (layer F.Cu) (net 7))
 (segment (start 24.892 -9.271) (end 25.146 -9.017) (width 0.508) (layer F.Cu) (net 7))
 (segment (start 32.385 12.954) (end 33.782 12.954) (width 0.508) (layer F.Cu) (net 16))
 (segment (start 33.782 12.954) (end 37.084 9.652) (width 0.508) (layer F.Cu) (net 16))
 (segment (start 37.084 9.652) (end 38.862 9.652) (width 0.508) (layer F.Cu) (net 16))
 (segment (start 38.862 9.652) (end 41.402 7.112) (width 0.508) (layer F.Cu) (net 16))
 (segment (start 41.402 7.112) (end 42.037 7.112) (width 0.508) (layer F.Cu) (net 16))
 (segment (start 30.353 -10.033) (end 30.353 -10.16) (width 0.508) (layer F.Cu) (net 4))
 (segment (start 30.353 -10.16) (end 29.083 -11.43) (width 0.508) (layer F.Cu) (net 4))
 (segment (start 19.431 -7.239) (end 19.05 -7.239) (width 0.508) (layer F.Cu) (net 29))
 (segment (start 19.05 -7.239) (end 17.653 -5.842) (width 0.508) (layer F.Cu) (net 29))
 (segment (start 17.653 -5.842) (end 17.653 -2.286) (width 0.508) (layer F.Cu) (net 29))
 (segment (start 19.05 -0.889) (end 19.05 -0.635) (width 0.508) (layer F.Cu) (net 16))
 (segment (start 19.05 -0.635) (end 20.955 1.27) (width 0.508) (layer F.Cu) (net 16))
 (segment (start 20.955 1.27) (end 22.987 1.27) (width 0.508) (layer F.Cu) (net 16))
 (segment (start 22.987 1.27) (end 27.051 -2.794) (width 0.508) (layer F.Cu) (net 16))
 (segment (start 27.051 -2.794) (end 27.051 -4.191) (width 0.508) (layer F.Cu) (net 16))
 (segment (start 27.051 -4.191) (end 25.781 -5.461) (width 0.508) (layer F.Cu) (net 16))
 (segment (start 24.892 -4.572) (end 24.003 -4.572) (width 0.508) (layer F.Cu) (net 1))
 (segment (start 24.003 -4.572) (end 20.955 -7.62) (width 0.508) (layer F.Cu) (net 1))
 (segment (start 20.955 -7.62) (end 20.955 -8.001) (width 0.508) (layer F.Cu) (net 1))
 (segment (start 20.955 -8.001) (end 19.431 -9.525) (width 0.508) (layer F.Cu) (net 1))
 (segment (start 19.431 -9.525) (end 19.431 -19.177) (width 0.508) (layer F.Cu) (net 1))
 (segment (start 23.876 8.509) (end 23.876 8.89) (width 0.508) (layer F.Cu) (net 16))
 (segment (start 23.876 8.89) (end 26.924 11.938) (width 0.508) (layer F.Cu) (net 16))
 (segment (start 26.924 11.938) (end 26.924 12.573) (width 0.508) (layer F.Cu) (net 16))
 (segment (start 26.924 12.573) (end 27.305 12.954) (width 0.508) (layer F.Cu) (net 16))
 (segment (start 27.305 12.954) (end 32.512 12.954) (width 0.508) (layer F.Cu) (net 16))
 (gr_line (start 22.86 -24.257) (end 43.18 -24.257) (angle 51566.20) (width 0.508) (layer Edge.Cuts))
 (gr_line (start 22.86 14.605) (end 43.18 14.605) (angle 51566.20) (width 0.508) (layer Edge.Cuts))
 (gr_line (start 16.51 -17.907) (end 16.51 8.255) (angle 51566.20) (width 0.508) (layer Edge.Cuts))
 (gr_line (start 49.53 -17.907) (end 49.53 8.255) (angle 51566.20) (width 0.508) (layer Edge.Cuts))
 (gr_line (start 22.86 -17.907) (end 22.86 -17.907) (angle -90.00) (width 0.508) (layer Edge.Cuts))
 (gr_line (start 43.18 -17.907) (end 43.18 -17.907) (angle -90.00) (width 0.508) (layer Edge.Cuts))
 (gr_line (start 43.18 8.255) (end 43.18 8.255) (angle -90.00) (width 0.508) (layer Edge.Cuts))
 (gr_line (start 22.86 8.255) (end 22.86 8.255) (angle -90.00) (width 0.508) (layer Edge.Cuts)))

